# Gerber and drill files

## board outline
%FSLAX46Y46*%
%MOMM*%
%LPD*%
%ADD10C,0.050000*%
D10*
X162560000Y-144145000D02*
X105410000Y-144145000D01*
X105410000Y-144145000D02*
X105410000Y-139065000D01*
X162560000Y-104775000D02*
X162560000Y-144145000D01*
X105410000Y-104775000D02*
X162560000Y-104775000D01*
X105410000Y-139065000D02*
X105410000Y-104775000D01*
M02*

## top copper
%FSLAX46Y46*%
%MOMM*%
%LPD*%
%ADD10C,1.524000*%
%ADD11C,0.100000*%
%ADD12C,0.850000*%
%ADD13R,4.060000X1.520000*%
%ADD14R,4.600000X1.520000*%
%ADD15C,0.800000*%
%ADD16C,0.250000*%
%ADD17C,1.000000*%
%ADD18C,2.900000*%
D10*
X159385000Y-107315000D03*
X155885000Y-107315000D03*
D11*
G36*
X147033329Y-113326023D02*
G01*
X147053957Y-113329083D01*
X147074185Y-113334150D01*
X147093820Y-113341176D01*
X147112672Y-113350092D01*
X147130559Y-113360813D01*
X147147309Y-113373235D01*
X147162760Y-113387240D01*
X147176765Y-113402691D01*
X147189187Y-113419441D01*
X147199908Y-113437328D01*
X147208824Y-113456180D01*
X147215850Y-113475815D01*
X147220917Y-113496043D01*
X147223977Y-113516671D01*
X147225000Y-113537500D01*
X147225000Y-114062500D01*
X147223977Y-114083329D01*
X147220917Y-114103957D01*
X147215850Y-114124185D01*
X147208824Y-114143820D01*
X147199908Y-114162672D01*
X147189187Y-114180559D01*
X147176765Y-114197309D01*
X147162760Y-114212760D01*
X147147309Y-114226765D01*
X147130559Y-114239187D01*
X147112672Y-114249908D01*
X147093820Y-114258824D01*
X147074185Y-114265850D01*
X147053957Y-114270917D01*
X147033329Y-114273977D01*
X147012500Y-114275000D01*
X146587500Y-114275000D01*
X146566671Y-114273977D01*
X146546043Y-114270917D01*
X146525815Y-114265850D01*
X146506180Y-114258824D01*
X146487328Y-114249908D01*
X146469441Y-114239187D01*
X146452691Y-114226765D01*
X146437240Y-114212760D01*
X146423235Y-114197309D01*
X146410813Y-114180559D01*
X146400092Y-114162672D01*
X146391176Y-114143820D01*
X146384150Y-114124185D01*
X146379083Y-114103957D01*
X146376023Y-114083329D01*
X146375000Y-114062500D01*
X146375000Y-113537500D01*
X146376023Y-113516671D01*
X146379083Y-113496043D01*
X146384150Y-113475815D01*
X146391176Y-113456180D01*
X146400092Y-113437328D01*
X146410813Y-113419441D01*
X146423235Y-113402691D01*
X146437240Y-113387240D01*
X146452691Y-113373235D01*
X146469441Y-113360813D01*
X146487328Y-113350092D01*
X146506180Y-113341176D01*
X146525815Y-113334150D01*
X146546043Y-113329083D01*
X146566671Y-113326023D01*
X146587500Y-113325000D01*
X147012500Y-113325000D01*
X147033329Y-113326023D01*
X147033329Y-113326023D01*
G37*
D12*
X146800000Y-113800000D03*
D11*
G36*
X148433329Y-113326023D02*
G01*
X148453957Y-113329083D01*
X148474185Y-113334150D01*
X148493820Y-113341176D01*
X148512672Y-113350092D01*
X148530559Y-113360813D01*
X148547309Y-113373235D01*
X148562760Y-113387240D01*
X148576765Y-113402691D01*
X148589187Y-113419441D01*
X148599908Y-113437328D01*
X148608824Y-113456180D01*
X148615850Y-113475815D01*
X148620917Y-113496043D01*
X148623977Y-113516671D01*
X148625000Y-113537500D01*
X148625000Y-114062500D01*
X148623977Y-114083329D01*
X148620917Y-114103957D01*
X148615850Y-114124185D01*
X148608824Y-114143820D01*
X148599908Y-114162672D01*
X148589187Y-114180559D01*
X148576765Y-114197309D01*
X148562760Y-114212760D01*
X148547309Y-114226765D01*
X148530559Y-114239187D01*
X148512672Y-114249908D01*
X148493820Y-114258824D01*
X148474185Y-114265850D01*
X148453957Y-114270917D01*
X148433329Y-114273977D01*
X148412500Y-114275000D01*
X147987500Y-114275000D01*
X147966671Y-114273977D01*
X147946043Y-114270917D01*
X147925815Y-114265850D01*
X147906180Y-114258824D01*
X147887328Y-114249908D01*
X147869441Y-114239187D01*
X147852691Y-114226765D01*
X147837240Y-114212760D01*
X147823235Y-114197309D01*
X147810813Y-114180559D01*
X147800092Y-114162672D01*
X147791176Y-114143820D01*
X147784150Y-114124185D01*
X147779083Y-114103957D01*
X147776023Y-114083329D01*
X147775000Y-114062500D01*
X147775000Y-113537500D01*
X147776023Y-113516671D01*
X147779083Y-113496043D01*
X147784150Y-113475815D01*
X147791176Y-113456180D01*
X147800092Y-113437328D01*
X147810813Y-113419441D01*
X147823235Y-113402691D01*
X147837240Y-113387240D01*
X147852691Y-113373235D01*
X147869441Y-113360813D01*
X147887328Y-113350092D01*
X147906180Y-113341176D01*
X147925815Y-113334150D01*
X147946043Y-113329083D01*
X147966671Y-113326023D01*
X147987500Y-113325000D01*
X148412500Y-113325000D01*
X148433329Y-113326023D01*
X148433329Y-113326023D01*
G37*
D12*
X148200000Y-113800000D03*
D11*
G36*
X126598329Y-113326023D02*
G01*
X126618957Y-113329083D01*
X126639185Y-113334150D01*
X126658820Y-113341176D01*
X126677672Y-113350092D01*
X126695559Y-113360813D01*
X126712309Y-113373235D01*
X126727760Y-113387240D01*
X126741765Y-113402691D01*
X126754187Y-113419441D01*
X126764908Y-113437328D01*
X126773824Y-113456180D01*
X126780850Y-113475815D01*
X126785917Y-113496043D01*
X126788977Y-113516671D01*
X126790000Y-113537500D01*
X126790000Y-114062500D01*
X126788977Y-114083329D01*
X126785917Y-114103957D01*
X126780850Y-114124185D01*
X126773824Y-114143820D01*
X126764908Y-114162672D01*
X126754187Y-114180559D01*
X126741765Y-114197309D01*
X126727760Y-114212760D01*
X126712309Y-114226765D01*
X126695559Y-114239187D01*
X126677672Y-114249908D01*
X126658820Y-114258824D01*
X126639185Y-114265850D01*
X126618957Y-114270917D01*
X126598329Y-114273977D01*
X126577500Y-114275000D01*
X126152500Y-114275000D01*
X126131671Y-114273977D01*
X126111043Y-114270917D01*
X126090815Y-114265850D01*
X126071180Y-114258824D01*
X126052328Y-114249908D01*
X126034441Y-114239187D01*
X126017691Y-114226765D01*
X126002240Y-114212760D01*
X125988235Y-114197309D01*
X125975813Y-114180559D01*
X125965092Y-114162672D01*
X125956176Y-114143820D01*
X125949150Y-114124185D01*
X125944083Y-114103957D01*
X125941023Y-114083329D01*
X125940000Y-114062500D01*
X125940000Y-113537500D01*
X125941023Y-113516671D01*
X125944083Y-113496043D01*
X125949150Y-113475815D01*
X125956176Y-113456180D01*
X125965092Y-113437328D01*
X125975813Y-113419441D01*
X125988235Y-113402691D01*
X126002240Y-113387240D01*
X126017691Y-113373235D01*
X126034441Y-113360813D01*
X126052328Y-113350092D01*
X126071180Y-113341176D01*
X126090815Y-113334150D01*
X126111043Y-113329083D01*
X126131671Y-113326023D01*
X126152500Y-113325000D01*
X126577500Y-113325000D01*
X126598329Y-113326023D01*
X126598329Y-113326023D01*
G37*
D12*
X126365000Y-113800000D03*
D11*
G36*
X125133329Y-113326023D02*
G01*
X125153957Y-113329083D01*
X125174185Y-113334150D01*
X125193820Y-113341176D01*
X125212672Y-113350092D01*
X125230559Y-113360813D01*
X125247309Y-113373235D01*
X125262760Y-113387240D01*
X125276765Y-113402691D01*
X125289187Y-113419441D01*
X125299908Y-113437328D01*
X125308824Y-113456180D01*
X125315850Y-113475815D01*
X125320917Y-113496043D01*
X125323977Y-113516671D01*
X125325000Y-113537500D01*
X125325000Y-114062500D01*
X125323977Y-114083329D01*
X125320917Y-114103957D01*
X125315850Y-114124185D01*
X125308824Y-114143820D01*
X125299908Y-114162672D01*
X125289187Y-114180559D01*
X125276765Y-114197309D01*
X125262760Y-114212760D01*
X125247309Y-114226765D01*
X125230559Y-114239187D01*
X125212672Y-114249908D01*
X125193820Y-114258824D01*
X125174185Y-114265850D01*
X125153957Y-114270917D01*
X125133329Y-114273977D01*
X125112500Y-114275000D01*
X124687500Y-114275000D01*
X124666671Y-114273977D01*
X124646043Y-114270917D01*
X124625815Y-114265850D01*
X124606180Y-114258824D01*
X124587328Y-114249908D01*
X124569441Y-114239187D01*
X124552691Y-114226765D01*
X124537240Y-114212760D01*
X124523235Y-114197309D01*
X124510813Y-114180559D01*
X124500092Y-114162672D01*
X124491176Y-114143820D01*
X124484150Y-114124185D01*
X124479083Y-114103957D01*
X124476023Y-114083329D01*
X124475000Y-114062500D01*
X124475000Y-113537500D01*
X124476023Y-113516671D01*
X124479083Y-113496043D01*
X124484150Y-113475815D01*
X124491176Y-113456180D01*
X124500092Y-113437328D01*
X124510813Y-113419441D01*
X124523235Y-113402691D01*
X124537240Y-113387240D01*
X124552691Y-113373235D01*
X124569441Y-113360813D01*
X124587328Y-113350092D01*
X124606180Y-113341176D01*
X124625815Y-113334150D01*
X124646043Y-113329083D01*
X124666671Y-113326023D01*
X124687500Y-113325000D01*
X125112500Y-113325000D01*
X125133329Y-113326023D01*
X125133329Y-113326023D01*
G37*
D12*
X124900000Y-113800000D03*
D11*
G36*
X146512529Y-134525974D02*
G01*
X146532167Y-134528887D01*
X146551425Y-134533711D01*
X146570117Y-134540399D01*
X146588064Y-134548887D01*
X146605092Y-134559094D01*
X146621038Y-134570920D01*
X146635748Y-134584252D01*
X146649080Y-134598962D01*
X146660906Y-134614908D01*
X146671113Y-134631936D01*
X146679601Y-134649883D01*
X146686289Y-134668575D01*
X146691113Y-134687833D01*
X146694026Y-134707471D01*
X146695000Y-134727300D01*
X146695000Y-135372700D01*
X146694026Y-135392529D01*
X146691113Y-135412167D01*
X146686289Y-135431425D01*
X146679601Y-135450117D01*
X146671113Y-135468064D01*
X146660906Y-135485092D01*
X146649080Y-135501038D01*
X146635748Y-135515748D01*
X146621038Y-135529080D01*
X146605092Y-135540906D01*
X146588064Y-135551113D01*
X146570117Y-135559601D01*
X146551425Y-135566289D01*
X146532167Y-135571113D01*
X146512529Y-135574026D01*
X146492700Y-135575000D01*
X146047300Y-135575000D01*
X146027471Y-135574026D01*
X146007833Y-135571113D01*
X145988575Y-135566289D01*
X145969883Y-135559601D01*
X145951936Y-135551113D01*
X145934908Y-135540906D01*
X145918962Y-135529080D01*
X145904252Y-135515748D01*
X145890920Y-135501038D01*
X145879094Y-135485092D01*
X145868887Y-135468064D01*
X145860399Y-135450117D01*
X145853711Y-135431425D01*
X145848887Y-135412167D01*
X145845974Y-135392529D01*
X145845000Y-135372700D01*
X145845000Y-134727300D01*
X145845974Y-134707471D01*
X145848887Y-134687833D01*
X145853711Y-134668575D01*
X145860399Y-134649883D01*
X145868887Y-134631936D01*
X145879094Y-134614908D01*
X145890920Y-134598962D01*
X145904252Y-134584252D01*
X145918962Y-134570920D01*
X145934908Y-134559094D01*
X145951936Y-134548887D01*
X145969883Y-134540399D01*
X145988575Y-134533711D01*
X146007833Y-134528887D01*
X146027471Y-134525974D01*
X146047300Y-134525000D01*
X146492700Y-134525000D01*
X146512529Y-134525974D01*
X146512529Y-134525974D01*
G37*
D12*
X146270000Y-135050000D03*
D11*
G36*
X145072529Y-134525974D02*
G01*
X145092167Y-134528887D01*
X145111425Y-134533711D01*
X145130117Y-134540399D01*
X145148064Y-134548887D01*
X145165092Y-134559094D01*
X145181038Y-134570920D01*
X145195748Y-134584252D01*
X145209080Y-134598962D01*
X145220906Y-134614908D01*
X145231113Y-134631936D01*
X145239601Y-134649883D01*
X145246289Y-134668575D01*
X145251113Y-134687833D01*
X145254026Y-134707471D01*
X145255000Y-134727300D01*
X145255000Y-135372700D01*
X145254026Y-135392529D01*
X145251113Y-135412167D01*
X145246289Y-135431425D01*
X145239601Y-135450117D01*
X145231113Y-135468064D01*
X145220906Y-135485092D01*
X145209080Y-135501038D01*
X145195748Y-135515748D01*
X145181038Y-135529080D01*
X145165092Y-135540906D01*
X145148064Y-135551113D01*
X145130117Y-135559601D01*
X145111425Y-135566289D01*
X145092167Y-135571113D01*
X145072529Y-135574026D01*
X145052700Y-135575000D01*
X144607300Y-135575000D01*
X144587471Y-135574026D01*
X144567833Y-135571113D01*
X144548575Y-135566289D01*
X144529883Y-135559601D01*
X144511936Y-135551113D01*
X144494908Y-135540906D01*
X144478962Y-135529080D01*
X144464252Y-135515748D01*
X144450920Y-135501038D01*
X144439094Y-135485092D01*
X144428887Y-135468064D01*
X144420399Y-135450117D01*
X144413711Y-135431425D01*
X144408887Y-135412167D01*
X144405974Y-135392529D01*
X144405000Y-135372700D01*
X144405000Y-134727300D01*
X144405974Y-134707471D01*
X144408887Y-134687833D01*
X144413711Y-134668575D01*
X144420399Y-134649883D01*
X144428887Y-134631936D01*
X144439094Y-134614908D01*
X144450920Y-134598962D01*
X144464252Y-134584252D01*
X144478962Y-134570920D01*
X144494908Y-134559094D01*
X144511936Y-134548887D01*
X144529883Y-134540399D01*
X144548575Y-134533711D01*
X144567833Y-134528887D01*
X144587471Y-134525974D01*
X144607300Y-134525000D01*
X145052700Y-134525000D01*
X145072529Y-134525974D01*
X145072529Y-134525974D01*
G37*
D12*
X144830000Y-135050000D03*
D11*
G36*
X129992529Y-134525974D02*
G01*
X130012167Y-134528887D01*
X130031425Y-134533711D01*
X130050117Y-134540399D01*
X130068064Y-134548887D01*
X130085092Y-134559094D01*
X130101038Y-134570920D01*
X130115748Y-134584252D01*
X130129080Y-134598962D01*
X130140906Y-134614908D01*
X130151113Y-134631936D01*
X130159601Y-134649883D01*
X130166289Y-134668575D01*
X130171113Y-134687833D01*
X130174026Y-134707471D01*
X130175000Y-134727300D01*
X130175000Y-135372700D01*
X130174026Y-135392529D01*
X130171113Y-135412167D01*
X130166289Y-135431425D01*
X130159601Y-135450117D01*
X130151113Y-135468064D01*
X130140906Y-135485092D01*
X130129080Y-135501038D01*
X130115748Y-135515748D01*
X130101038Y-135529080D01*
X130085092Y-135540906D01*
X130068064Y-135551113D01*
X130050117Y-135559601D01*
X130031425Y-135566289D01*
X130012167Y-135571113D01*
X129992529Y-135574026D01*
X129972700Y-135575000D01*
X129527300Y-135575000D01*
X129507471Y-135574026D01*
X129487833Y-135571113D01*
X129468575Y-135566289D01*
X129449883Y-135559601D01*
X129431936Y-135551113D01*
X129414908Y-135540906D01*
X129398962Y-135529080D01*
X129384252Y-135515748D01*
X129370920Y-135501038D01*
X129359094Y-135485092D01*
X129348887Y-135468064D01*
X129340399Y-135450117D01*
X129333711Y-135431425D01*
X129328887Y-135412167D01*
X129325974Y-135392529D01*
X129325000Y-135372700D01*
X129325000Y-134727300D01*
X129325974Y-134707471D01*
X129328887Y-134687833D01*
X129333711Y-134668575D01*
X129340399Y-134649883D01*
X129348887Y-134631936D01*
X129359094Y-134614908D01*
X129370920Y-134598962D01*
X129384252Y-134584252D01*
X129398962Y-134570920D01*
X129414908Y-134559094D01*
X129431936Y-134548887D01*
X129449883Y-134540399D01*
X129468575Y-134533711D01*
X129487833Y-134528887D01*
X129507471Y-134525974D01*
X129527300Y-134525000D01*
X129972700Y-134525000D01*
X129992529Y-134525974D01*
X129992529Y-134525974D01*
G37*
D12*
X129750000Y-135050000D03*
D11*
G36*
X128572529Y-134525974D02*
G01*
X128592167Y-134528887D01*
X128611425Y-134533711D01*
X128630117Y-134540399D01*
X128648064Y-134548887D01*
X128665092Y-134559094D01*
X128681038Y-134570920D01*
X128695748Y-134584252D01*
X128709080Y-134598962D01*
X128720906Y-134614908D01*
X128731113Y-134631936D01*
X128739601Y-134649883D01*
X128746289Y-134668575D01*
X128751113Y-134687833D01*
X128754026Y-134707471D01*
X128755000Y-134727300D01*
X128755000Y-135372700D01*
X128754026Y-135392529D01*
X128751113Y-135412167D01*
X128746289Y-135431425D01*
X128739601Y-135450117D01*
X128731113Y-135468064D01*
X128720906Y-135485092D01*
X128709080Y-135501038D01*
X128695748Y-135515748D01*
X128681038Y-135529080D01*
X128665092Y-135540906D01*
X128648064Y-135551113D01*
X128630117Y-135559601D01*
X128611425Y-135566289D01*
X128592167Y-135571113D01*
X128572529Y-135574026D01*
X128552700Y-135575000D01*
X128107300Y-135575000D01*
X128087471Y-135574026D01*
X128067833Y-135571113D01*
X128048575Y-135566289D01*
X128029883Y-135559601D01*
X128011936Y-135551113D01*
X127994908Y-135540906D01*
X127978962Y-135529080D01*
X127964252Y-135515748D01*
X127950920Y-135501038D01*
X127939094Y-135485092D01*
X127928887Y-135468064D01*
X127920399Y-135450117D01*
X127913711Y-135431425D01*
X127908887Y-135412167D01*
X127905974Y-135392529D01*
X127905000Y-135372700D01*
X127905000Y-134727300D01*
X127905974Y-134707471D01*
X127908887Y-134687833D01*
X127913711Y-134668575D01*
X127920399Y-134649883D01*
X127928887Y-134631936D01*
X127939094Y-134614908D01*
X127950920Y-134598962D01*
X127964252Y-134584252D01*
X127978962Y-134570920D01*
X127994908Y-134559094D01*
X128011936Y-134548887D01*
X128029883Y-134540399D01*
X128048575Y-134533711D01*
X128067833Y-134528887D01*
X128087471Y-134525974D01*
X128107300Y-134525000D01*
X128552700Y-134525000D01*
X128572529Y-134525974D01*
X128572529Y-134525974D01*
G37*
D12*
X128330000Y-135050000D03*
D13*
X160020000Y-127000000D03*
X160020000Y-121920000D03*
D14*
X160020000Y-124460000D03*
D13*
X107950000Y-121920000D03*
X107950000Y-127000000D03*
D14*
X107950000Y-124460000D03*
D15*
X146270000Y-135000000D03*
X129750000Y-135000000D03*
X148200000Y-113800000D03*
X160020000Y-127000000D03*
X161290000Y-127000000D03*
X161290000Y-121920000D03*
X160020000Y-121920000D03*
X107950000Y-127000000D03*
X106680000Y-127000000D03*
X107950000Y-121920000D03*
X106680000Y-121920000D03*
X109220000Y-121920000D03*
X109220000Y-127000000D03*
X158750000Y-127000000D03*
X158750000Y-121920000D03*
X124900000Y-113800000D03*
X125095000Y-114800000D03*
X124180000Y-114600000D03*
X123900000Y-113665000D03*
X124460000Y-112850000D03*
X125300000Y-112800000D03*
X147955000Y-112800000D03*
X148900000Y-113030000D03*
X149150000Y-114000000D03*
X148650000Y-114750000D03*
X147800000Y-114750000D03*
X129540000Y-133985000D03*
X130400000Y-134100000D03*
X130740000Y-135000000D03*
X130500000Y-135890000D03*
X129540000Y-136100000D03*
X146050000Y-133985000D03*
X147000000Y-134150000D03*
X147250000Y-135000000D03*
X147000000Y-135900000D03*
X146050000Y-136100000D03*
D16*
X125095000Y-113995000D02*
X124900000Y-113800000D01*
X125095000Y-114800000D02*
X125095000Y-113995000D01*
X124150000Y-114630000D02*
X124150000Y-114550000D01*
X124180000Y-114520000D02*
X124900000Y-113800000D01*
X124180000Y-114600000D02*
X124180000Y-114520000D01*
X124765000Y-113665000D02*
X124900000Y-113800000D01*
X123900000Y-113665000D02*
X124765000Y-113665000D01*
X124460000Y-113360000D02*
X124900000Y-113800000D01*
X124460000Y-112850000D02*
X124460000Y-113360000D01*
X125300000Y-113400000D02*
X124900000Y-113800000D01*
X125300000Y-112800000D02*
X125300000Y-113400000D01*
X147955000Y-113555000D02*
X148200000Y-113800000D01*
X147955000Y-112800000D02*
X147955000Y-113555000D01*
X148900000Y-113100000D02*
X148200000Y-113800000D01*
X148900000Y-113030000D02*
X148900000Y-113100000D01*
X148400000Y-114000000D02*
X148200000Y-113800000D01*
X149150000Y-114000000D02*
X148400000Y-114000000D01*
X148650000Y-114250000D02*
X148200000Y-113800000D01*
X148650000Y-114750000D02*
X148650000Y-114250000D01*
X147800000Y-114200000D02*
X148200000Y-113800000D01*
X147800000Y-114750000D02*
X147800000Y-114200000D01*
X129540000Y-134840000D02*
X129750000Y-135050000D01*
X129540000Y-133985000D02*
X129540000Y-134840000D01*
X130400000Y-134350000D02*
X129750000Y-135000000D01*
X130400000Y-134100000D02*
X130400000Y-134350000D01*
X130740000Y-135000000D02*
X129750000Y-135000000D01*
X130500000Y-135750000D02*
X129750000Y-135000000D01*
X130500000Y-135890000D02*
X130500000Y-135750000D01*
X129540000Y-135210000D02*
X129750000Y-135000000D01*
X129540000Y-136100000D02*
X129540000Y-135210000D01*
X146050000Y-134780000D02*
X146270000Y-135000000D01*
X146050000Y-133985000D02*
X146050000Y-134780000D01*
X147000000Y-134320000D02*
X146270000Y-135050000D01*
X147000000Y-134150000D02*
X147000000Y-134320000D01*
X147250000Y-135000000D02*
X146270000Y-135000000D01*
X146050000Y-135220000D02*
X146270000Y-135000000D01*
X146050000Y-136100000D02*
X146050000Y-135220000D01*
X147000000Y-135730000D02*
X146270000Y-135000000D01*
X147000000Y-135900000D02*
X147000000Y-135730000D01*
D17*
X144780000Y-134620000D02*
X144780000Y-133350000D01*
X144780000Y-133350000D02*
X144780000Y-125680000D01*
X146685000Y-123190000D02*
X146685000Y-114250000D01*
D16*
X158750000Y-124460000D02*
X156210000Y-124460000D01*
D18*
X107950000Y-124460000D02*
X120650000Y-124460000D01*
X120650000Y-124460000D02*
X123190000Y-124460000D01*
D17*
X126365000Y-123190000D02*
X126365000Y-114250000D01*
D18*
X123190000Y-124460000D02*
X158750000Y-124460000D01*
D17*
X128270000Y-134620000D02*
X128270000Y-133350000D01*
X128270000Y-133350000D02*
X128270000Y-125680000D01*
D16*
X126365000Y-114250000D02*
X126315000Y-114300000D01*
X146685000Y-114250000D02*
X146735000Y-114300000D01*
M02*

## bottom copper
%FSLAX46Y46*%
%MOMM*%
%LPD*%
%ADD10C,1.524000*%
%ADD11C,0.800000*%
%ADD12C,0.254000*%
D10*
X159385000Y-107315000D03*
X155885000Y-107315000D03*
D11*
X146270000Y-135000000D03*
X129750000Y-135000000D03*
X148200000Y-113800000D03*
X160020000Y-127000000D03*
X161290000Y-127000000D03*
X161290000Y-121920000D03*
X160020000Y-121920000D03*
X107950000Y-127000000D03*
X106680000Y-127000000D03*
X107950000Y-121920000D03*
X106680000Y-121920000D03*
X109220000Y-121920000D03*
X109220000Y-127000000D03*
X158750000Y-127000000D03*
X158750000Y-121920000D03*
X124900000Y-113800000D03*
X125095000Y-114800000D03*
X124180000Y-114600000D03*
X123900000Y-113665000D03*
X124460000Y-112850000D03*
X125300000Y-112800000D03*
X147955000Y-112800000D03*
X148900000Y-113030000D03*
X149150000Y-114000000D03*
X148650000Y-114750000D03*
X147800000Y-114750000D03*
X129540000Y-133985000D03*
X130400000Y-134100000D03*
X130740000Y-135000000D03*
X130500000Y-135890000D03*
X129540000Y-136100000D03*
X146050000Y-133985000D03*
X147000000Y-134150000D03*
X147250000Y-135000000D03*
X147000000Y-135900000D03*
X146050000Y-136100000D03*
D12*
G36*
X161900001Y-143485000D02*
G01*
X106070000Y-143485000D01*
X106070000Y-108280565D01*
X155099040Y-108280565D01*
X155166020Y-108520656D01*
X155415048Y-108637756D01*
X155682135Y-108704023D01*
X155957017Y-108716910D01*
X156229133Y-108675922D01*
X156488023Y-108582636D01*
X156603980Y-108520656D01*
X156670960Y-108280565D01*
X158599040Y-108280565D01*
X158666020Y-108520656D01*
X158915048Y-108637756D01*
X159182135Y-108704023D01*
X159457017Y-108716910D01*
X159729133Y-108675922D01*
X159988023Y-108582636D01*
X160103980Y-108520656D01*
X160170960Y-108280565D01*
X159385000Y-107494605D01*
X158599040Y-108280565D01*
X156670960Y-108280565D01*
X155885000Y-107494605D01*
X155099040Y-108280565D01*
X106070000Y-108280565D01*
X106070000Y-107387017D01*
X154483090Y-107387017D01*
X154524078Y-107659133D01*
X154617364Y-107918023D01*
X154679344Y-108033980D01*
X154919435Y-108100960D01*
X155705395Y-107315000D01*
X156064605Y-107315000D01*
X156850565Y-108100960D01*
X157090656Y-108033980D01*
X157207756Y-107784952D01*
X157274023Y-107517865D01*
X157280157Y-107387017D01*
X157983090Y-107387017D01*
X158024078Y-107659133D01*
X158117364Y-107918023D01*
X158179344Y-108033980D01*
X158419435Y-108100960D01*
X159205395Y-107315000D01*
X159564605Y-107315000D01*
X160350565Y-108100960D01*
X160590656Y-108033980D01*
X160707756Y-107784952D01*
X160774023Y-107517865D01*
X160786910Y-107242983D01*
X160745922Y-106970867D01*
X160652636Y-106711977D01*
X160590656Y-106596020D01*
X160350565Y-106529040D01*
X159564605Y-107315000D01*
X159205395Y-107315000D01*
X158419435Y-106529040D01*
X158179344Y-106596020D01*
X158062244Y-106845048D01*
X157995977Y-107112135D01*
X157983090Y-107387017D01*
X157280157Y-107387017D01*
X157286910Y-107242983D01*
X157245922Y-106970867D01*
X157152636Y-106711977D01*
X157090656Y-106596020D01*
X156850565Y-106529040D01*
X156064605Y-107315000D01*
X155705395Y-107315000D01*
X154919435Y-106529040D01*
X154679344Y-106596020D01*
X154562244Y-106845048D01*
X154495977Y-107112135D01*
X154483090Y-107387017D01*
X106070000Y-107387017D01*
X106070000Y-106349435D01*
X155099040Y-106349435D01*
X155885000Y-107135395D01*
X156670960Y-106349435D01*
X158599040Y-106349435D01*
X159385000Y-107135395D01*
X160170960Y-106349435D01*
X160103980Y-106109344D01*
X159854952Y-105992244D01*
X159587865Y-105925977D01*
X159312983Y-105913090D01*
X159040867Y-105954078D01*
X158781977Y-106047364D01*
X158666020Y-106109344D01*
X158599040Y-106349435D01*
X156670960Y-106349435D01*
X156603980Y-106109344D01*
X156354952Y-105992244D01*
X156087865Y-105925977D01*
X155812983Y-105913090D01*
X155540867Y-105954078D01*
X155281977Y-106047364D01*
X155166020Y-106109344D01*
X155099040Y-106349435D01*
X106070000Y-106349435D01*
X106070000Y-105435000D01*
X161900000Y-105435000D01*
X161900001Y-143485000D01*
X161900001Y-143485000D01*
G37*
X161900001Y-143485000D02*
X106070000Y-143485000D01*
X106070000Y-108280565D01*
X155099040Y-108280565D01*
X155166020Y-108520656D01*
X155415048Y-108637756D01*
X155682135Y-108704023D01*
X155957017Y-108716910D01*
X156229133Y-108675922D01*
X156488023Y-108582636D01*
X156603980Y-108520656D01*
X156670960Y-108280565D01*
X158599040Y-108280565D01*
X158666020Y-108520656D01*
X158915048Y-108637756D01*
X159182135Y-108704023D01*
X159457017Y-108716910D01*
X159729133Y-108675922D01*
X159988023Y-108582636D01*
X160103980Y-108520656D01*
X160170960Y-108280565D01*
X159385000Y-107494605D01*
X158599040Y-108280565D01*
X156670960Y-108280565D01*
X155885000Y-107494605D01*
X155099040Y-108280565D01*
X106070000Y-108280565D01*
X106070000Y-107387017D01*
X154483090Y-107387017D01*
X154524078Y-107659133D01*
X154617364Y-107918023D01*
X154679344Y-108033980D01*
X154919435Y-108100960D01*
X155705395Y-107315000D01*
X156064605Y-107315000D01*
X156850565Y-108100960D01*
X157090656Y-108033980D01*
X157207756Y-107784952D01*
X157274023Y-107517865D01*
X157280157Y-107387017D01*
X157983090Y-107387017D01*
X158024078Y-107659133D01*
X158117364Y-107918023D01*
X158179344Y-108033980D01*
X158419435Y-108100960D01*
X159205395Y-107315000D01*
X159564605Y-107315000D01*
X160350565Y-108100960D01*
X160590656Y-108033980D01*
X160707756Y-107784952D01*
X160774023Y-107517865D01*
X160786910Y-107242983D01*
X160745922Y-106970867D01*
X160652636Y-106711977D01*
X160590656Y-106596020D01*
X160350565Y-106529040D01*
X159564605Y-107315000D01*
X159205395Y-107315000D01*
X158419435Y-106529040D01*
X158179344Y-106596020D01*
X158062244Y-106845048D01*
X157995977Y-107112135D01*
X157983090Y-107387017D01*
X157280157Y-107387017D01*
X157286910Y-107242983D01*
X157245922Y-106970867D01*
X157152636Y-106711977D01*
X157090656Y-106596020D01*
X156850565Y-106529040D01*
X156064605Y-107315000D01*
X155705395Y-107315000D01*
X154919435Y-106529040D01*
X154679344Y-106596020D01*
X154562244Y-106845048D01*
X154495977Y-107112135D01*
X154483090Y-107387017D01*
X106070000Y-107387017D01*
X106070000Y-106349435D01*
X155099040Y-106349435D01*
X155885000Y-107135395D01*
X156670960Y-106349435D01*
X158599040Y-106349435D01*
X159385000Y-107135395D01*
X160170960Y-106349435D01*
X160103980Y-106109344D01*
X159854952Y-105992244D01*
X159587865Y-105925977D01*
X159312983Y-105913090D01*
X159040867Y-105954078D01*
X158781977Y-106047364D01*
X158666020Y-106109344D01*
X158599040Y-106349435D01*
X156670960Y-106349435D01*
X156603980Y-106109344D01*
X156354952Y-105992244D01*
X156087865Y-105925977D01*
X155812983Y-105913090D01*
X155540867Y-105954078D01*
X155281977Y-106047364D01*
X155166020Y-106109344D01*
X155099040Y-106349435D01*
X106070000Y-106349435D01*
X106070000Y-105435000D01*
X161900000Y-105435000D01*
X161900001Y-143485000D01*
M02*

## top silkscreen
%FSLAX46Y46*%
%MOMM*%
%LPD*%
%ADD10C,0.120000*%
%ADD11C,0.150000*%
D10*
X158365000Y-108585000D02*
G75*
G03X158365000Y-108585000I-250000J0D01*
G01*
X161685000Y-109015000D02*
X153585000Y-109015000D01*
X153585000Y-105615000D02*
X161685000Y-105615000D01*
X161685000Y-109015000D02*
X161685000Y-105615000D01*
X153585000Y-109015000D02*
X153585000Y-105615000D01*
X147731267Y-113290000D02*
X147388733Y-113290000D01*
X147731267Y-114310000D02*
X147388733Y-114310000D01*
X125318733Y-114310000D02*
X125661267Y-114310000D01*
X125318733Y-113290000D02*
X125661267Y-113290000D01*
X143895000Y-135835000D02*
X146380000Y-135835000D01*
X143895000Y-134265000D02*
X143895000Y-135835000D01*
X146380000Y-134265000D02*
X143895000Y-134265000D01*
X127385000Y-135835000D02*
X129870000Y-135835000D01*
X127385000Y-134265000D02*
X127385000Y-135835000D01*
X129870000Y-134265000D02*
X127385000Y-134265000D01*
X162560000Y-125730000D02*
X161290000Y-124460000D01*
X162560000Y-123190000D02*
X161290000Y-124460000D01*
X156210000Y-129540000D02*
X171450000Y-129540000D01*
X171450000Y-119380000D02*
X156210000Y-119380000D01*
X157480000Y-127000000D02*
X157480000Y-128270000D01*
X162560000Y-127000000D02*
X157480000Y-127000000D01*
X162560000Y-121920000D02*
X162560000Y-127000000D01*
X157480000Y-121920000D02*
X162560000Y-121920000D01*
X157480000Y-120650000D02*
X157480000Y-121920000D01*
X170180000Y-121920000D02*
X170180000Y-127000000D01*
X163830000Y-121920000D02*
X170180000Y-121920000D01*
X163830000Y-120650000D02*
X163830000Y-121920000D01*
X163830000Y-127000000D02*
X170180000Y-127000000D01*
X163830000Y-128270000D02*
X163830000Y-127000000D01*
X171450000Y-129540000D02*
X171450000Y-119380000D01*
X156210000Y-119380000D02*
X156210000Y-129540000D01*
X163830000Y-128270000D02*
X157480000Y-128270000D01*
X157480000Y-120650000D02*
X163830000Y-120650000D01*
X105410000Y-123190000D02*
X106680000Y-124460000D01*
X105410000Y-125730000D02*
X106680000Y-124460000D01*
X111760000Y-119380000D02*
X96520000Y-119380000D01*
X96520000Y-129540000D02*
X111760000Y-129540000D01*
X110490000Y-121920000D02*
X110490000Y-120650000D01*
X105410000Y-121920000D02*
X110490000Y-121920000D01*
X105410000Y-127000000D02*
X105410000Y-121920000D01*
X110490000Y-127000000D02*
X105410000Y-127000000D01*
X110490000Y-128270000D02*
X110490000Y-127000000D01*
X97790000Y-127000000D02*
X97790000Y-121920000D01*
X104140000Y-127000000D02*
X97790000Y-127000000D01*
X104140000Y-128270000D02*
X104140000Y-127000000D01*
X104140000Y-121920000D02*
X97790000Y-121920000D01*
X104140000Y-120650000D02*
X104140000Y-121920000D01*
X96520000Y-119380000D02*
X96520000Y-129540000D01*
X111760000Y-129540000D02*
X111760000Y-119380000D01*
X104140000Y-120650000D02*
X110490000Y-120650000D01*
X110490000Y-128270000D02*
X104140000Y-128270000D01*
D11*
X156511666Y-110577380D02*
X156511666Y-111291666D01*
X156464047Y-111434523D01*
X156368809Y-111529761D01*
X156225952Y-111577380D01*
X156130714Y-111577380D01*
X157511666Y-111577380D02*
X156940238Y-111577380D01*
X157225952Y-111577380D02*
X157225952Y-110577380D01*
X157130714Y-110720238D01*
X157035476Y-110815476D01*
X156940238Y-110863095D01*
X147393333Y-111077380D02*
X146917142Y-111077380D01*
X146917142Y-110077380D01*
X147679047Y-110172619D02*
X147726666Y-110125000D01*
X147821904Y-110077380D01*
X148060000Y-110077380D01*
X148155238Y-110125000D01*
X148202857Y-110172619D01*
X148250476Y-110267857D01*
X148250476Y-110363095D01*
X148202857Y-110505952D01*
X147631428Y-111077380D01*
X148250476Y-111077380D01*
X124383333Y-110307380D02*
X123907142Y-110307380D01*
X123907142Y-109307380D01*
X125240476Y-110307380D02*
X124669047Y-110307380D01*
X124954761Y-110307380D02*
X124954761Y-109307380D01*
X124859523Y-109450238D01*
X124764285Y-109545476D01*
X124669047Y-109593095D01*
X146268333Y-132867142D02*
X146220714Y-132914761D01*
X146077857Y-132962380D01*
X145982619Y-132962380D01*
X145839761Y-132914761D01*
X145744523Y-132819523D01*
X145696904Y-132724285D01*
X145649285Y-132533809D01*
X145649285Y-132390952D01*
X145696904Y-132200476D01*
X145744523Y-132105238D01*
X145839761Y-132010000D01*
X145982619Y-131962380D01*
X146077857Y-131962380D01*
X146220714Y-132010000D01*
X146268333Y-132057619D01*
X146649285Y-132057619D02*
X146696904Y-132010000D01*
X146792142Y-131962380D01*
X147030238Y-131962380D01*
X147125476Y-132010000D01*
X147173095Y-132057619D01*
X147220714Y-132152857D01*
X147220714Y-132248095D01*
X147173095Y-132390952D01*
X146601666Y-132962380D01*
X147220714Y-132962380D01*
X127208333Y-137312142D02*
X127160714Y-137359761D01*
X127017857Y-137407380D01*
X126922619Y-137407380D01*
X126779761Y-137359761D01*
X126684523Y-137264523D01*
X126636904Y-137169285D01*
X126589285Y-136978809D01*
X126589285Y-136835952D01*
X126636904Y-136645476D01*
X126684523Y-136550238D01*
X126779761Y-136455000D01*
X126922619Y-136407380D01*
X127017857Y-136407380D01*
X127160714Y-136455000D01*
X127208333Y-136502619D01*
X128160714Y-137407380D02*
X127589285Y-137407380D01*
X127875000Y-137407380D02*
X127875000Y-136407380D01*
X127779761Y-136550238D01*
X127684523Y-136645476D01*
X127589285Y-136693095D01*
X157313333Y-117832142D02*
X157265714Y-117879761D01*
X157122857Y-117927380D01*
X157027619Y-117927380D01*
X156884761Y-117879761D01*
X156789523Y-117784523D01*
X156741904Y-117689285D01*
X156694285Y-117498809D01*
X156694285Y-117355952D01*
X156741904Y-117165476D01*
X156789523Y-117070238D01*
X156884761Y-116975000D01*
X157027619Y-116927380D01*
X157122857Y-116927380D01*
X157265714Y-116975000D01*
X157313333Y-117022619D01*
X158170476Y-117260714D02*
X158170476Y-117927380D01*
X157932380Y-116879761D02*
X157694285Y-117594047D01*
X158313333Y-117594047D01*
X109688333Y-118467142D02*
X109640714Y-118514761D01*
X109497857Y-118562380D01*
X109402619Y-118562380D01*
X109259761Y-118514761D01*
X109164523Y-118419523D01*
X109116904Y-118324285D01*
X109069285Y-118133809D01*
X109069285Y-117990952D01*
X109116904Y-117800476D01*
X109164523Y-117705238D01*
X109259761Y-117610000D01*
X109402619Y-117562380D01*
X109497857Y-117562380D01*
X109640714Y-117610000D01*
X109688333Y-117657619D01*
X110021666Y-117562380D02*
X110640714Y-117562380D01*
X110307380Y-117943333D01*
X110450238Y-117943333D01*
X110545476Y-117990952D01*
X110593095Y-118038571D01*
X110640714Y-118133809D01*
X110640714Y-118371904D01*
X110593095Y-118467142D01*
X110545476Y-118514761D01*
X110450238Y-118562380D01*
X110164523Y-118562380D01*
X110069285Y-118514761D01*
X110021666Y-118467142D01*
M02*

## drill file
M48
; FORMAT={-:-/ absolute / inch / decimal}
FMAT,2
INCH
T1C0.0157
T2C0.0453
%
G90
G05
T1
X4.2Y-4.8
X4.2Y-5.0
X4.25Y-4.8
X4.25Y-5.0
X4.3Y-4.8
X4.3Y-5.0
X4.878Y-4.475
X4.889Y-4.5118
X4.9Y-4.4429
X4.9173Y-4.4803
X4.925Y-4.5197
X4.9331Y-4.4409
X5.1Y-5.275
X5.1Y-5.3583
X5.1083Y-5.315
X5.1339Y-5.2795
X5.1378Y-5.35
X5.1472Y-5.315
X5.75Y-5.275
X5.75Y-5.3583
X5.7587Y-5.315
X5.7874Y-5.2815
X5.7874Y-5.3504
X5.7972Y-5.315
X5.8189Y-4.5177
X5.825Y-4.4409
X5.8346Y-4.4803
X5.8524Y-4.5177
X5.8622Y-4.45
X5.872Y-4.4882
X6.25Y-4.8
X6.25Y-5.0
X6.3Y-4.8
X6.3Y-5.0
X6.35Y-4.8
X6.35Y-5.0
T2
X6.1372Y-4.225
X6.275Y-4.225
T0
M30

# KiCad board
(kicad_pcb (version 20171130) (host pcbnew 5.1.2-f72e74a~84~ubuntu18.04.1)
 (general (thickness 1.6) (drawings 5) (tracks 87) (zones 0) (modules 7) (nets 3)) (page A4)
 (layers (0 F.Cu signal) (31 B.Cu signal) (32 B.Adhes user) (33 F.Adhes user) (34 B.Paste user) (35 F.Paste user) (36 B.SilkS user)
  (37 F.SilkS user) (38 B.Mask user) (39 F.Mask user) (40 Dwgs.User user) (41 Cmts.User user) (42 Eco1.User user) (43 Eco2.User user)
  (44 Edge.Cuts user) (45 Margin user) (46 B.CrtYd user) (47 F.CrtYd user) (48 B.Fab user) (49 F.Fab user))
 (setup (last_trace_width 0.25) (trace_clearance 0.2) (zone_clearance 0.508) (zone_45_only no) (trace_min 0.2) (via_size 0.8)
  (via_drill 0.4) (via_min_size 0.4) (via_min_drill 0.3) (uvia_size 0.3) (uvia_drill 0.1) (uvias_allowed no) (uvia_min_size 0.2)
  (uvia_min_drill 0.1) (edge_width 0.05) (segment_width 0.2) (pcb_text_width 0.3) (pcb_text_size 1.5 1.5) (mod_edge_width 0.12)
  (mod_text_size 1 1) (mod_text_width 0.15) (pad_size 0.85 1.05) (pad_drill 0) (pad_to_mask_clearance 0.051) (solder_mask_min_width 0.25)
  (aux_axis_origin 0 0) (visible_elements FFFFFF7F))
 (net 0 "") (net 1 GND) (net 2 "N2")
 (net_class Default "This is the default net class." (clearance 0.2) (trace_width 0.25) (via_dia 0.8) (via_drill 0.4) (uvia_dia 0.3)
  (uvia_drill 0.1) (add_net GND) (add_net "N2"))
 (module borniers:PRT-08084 (layer F.Cu) (at 159.385 112.395)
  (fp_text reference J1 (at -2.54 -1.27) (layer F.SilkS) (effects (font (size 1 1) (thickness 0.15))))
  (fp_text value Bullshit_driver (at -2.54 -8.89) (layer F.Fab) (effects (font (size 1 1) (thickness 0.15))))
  (fp_circle (center -1.27 -3.81) (end -1.02 -3.81) (layer F.SilkS) (width 0.12))
  (fp_line (start 2.3 -3.38) (end -5.8 -3.38) (layer F.SilkS) (width 0.12))
  (fp_line (start -5.8 -6.78) (end 2.3 -6.78) (layer F.SilkS) (width 0.12))
  (fp_line (start 2.3 -3.38) (end 2.3 -6.78) (layer F.SilkS) (width 0.12))
  (fp_line (start -5.8 -3.38) (end -5.8 -6.78) (layer F.SilkS) (width 0.12))
  (pad 2 thru_hole circle (at 0 -5.08) (size 1.524 1.524) (drill 1.15) (layers *.Cu *.Mask) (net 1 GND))
  (pad 1 thru_hole circle (at -3.5 -5.08) (size 1.524 1.524) (drill 1.15) (layers *.Cu *.Mask) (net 1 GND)))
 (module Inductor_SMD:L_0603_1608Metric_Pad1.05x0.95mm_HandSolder (layer F.Cu) (at 147.56 113.8 180)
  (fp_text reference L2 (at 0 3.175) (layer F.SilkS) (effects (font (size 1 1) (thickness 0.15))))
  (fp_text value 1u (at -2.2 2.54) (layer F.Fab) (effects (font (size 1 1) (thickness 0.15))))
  (fp_line (start -0.171267 0.51) (end 0.171267 0.51) (layer F.SilkS) (width 0.12))
  (fp_line (start -0.171267 -0.51) (end 0.171267 -0.51) (layer F.SilkS) (width 0.12))
  (pad 2 smd roundrect (at 0.76 0 180) (size 0.85 0.95) (layers F.Cu F.Paste F.Mask) (roundrect_rratio 0.25) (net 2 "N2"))
  (pad 1 smd roundrect (at -0.64 0 180) (size 0.85 0.95) (layers F.Cu F.Paste F.Mask) (roundrect_rratio 0.25) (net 1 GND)))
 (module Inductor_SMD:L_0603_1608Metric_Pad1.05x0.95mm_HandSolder (layer F.Cu) (at 125.49 113.8)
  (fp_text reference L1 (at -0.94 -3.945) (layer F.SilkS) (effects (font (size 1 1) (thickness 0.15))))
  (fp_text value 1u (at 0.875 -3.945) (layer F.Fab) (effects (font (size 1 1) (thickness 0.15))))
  (fp_line (start -0.171267 0.51) (end 0.171267 0.51) (layer F.SilkS) (width 0.12))
  (fp_line (start -0.171267 -0.51) (end 0.171267 -0.51) (layer F.SilkS) (width 0.12))
  (pad 2 smd roundrect (at 0.875 0) (size 0.85 0.95) (layers F.Cu F.Paste F.Mask) (roundrect_rratio 0.25) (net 2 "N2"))
  (pad 1 smd roundrect (at -0.59 0) (size 0.85 0.95) (layers F.Cu F.Paste F.Mask) (roundrect_rratio 0.25) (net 1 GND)))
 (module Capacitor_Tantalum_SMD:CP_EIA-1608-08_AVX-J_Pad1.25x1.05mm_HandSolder (layer F.Cu) (at 145.58 135.05)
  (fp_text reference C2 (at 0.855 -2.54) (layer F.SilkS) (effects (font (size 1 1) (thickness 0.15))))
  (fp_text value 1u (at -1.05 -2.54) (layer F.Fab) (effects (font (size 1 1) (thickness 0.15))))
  (fp_line (start -1.685 0.785) (end 0.8 0.785) (layer F.SilkS) (width 0.12))
  (fp_line (start -1.685 -0.785) (end -1.685 0.785) (layer F.SilkS) (width 0.12))
  (fp_line (start 0.8 -0.785) (end -1.685 -0.785) (layer F.SilkS) (width 0.12))
  (pad 2 smd roundrect (at 0.69 0) (size 0.85 1.05) (layers F.Cu F.Paste F.Mask) (roundrect_rratio 0.238) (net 1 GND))
  (pad 1 smd roundrect (at -0.75 0) (size 0.85 1.05) (layers F.Cu F.Paste F.Mask) (roundrect_rratio 0.238) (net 2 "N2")))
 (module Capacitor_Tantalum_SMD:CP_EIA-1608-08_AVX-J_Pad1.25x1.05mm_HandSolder (layer F.Cu) (at 129.07 135.05)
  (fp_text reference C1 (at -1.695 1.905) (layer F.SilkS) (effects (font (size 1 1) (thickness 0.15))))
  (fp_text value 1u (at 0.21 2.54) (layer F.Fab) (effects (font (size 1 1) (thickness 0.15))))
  (fp_line (start -1.685 0.785) (end 0.8 0.785) (layer F.SilkS) (width 0.12))
  (fp_line (start -1.685 -0.785) (end -1.685 0.785) (layer F.SilkS) (width 0.12))
  (fp_line (start 0.8 -0.785) (end -1.685 -0.785) (layer F.SilkS) (width 0.12))
  (pad 2 smd roundrect (at 0.68 0) (size 0.85 1.05) (layers F.Cu F.Paste F.Mask) (roundrect_rratio 0.238) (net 1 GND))
  (pad 1 smd roundrect (at -0.74 0) (size 0.85 1.05) (layers F.Cu F.Paste F.Mask) (roundrect_rratio 0.238) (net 2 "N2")))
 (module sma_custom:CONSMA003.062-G (layer F.Cu) (at 163.83 127)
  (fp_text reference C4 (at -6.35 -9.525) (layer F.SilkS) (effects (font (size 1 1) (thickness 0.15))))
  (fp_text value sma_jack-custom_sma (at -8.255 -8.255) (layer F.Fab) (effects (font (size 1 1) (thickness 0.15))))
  (fp_line (start -1.27 -1.27) (end -2.54 -2.54) (layer F.SilkS) (width 0.12))
  (fp_line (start -1.27 -3.81) (end -2.54 -2.54) (layer F.SilkS) (width 0.12))
  (fp_line (start -7.62 2.54) (end 7.62 2.54) (layer F.SilkS) (width 0.12))
  (fp_line (start 7.62 -7.62) (end -7.62 -7.62) (layer F.SilkS) (width 0.12))
  (fp_line (start -6.35 0) (end -6.35 1.27) (layer F.SilkS) (width 0.12))
  (fp_line (start -1.27 0) (end -6.35 0) (layer F.SilkS) (width 0.12))
  (fp_line (start -1.27 -5.08) (end -1.27 0) (layer F.SilkS) (width 0.12))
  (fp_line (start -6.35 -5.08) (end -1.27 -5.08) (layer F.SilkS) (width 0.12))
  (fp_line (start -6.35 -6.35) (end -6.35 -5.08) (layer F.SilkS) (width 0.12))
  (fp_line (start 6.35 -5.08) (end 6.35 0) (layer F.SilkS) (width 0.12))
  (fp_line (start 0 -5.08) (end 6.35 -5.08) (layer F.SilkS) (width 0.12))
  (fp_line (start 0 -6.35) (end 0 -5.08) (layer F.SilkS) (width 0.12))
  (fp_line (start 0 0) (end 6.35 0) (layer F.SilkS) (width 0.12))
  (fp_line (start 0 1.27) (end 0 0) (layer F.SilkS) (width 0.12))
  (fp_line (start 7.62 2.54) (end 7.62 -7.62) (layer F.SilkS) (width 0.12))
  (fp_line (start -7.62 -7.62) (end -7.62 2.54) (layer F.SilkS) (width 0.12))
  (fp_line (start 0 1.27) (end -6.35 1.27) (layer F.SilkS) (width 0.12))
  (fp_line (start -6.35 -6.35) (end 0 -6.35) (layer F.SilkS) (width 0.12))
  (pad 3 smd rect (at -3.81 0) (size 4.06 1.52) (layers F.Cu F.Paste F.Mask) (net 1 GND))
  (pad 2 smd rect (at -3.81 -5.08) (size 4.06 1.52) (layers F.Cu F.Paste F.Mask) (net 1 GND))
  (pad 1 smd rect (at -3.81 -2.54) (size 4.6 1.52) (layers F.Cu F.Paste F.Mask) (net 2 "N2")))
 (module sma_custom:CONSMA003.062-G (layer F.Cu) (at 104.14 121.92 180)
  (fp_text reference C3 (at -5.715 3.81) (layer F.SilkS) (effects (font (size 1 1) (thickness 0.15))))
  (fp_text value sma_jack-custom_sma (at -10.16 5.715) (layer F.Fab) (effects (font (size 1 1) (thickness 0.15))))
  (fp_line (start -1.27 -1.27) (end -2.54 -2.54) (layer F.SilkS) (width 0.12))
  (fp_line (start -1.27 -3.81) (end -2.54 -2.54) (layer F.SilkS) (width 0.12))
  (fp_line (start -7.62 2.54) (end 7.62 2.54) (layer F.SilkS) (width 0.12))
  (fp_line (start 7.62 -7.62) (end -7.62 -7.62) (layer F.SilkS) (width 0.12))
  (fp_line (start -6.35 0) (end -6.35 1.27) (layer F.SilkS) (width 0.12))
  (fp_line (start -1.27 0) (end -6.35 0) (layer F.SilkS) (width 0.12))
  (fp_line (start -1.27 -5.08) (end -1.27 0) (layer F.SilkS) (width 0.12))
  (fp_line (start -6.35 -5.08) (end -1.27 -5.08) (layer F.SilkS) (width 0.12))
  (fp_line (start -6.35 -6.35) (end -6.35 -5.08) (layer F.SilkS) (width 0.12))
  (fp_line (start 6.35 -5.08) (end 6.35 0) (layer F.SilkS) (width 0.12))
  (fp_line (start 0 -5.08) (end 6.35 -5.08) (layer F.SilkS) (width 0.12))
  (fp_line (start 0 -6.35) (end 0 -5.08) (layer F.SilkS) (width 0.12))
  (fp_line (start 0 0) (end 6.35 0) (layer F.SilkS) (width 0.12))
  (fp_line (start 0 1.27) (end 0 0) (layer F.SilkS) (width 0.12))
  (fp_line (start 7.62 2.54) (end 7.62 -7.62) (layer F.SilkS) (width 0.12))
  (fp_line (start -7.62 -7.62) (end -7.62 2.54) (layer F.SilkS) (width 0.12))
  (fp_line (start 0 1.27) (end -6.35 1.27) (layer F.SilkS) (width 0.12))
  (fp_line (start -6.35 -6.35) (end 0 -6.35) (layer F.SilkS) (width 0.12))
  (pad 3 smd rect (at -3.81 0 180) (size 4.06 1.52) (layers F.Cu F.Paste F.Mask) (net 1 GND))
  (pad 2 smd rect (at -3.81 -5.08 180) (size 4.06 1.52) (layers F.Cu F.Paste F.Mask) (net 1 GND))
  (pad 1 smd rect (at -3.81 -2.54 180) (size 4.6 1.52) (layers F.Cu F.Paste F.Mask) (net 2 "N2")))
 (gr_line (start 162.56 144.145) (end 105.41 144.145) (layer Edge.Cuts) (width 0.05))
 (gr_line (start 105.41 144.145) (end 105.41 139.065) (layer Edge.Cuts) (width 0.05))
 (gr_line (start 162.56 104.775) (end 162.56 144.145) (layer Edge.Cuts) (width 0.05))
 (gr_line (start 105.41 104.775) (end 162.56 104.775) (layer Edge.Cuts) (width 0.05))
 (gr_line (start 105.41 139.065) (end 105.41 104.775) (layer Edge.Cuts) (width 0.05))
 (via (at 146.27 135) (size 0.8) (drill 0.4) (layers F.Cu B.Cu) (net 1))
 (via (at 129.75 135) (size 0.8) (drill 0.4) (layers F.Cu B.Cu) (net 1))
 (via (at 148.2 113.8) (size 0.8) (drill 0.4) (layers F.Cu B.Cu) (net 1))
 (via (at 160.02 127) (size 0.8) (drill 0.4) (layers F.Cu B.Cu) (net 1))
 (via (at 161.29 127) (size 0.8) (drill 0.4) (layers F.Cu B.Cu) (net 1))
 (via (at 161.29 121.92) (size 0.8) (drill 0.4) (layers F.Cu B.Cu) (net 1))
 (via (at 160.02 121.92) (size 0.8) (drill 0.4) (layers F.Cu B.Cu) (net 1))
 (via (at 107.95 127) (size 0.8) (drill 0.4) (layers F.Cu B.Cu) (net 1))
 (via (at 106.68 127) (size 0.8) (drill 0.4) (layers F.Cu B.Cu) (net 1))
 (via (at 107.95 121.92) (size 0.8) (drill 0.4) (layers F.Cu B.Cu) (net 1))
 (via (at 106.68 121.92) (size 0.8) (drill 0.4) (layers F.Cu B.Cu) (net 1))
 (via (at 109.22 121.92) (size 0.8) (drill 0.4) (layers F.Cu B.Cu) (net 1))
 (via (at 109.22 127) (size 0.8) (drill 0.4) (layers F.Cu B.Cu) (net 1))
 (via (at 158.75 127) (size 0.8) (drill 0.4) (layers F.Cu B.Cu) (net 1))
 (via (at 158.75 121.92) (size 0.8) (drill 0.4) (layers F.Cu B.Cu) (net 1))
 (via (at 124.9 113.8) (size 0.8) (drill 0.4) (layers F.Cu B.Cu) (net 1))
 (via (at 125.095 114.8) (size 0.8) (drill 0.4) (layers F.Cu B.Cu) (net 1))
 (segment (start 125.095 113.995) (end 124.9 113.8) (width 0.25) (layer F.Cu) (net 1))
 (segment (start 125.095 114.8) (end 125.095 113.995) (width 0.25) (layer F.Cu) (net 1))
 (via (at 124.18 114.6) (size 0.8) (drill 0.4) (layers F.Cu B.Cu) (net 1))
 (segment (start 124.15 114.63) (end 124.15 114.55) (width 0.25) (layer F.Cu) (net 1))
 (segment (start 124.18 114.52) (end 124.9 113.8) (width 0.25) (layer F.Cu) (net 1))
 (segment (start 124.18 114.6) (end 124.18 114.52) (width 0.25) (layer F.Cu) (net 1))
 (via (at 123.9 113.665) (size 0.8) (drill 0.4) (layers F.Cu B.Cu) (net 1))
 (segment (start 124.765 113.665) (end 124.9 113.8) (width 0.25) (layer F.Cu) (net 1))
 (segment (start 123.9 113.665) (end 124.765 113.665) (width 0.25) (layer F.Cu) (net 1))
 (via (at 124.46 112.85) (size 0.8) (drill 0.4) (layers F.Cu B.Cu) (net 1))
 (segment (start 124.46 113.36) (end 124.9 113.8) (width 0.25) (layer F.Cu) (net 1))
 (segment (start 124.46 112.85) (end 124.46 113.36) (width 0.25) (layer F.Cu) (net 1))
 (via (at 125.3 112.8) (size 0.8) (drill 0.4) (layers F.Cu B.Cu) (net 1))
 (segment (start 125.3 113.4) (end 124.9 113.8) (width 0.25) (layer F.Cu) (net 1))
 (segment (start 125.3 112.8) (end 125.3 113.4) (width 0.25) (layer F.Cu) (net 1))
 (via (at 147.955 112.8) (size 0.8) (drill 0.4) (layers F.Cu B.Cu) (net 1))
 (via (at 148.9 113.03) (size 0.8) (drill 0.4) (layers F.Cu B.Cu) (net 1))
 (via (at 149.15 114) (size 0.8) (drill 0.4) (layers F.Cu B.Cu) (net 1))
 (via (at 148.65 114.75) (size 0.8) (drill 0.4) (layers F.Cu B.Cu) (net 1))
 (segment (start 147.955 113.555) (end 148.2 113.8) (width 0.25) (layer F.Cu) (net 1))
 (segment (start 147.955 112.8) (end 147.955 113.555) (width 0.25) (layer F.Cu) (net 1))
 (segment (start 148.9 113.1) (end 148.2 113.8) (width 0.25) (layer F.Cu) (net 1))
 (segment (start 148.9 113.03) (end 148.9 113.1) (width 0.25) (layer F.Cu) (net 1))
 (segment (start 148.4 114) (end 148.2 113.8) (width 0.25) (layer F.Cu) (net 1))
 (segment (start 149.15 114) (end 148.4 114) (width 0.25) (layer F.Cu) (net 1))
 (segment (start 148.65 114.25) (end 148.2 113.8) (width 0.25) (layer F.Cu) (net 1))
 (segment (start 148.65 114.75) (end 148.65 114.25) (width 0.25) (layer F.Cu) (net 1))
 (via (at 147.8 114.75) (size 0.8) (drill 0.4) (layers F.Cu B.Cu) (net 1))
 (segment (start 147.8 114.2) (end 148.2 113.8) (width 0.25) (layer F.Cu) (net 1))
 (segment (start 147.8 114.75) (end 147.8 114.2) (width 0.25) (layer F.Cu) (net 1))
 (via (at 129.54 133.985) (size 0.8) (drill 0.4) (layers F.Cu B.Cu) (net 1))
 (via (at 130.4 134.1) (size 0.8) (drill 0.4) (layers F.Cu B.Cu) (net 1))
 (via (at 130.74 135) (size 0.8) (drill 0.4) (layers F.Cu B.Cu) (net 1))
 (via (at 130.5 135.89) (size 0.8) (drill 0.4) (layers F.Cu B.Cu) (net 1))
 (via (at 129.54 136.1) (size 0.8) (drill 0.4) (layers F.Cu B.Cu) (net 1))
 (segment (start 129.54 134.84) (end 129.75 135.05) (width 0.25) (layer F.Cu) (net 1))
 (segment (start 129.54 133.985) (end 129.54 134.84) (width 0.25) (layer F.Cu) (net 1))
 (segment (start 130.4 134.35) (end 129.75 135) (width 0.25) (layer F.Cu) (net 1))
 (segment (start 130.4 134.1) (end 130.4 134.35) (width 0.25) (layer F.Cu) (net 1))
 (segment (start 130.74 135) (end 129.75 135) (width 0.25) (layer F.Cu) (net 1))
 (segment (start 130.5 135.75) (end 129.75 135) (width 0.25) (layer F.Cu) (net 1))
 (segment (start 130.5 135.89) (end 130.5 135.75) (width 0.25) (layer F.Cu) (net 1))
 (segment (start 129.54 135.21) (end 129.75 135) (width 0.25) (layer F.Cu) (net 1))
 (segment (start 129.54 136.1) (end 129.54 135.21) (width 0.25) (layer F.Cu) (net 1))
 (via (at 146.05 133.985) (size 0.8) (drill 0.4) (layers F.Cu B.Cu) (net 1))
 (via (at 147 134.15) (size 0.8) (drill 0.4) (layers F.Cu B.Cu) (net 1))
 (via (at 147.25 135) (size 0.8) (drill 0.4) (layers F.Cu B.Cu) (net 1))
 (via (at 147 135.9) (size 0.8) (drill 0.4) (layers F.Cu B.Cu) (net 1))
 (via (at 146.05 136.1) (size 0.8) (drill 0.4) (layers F.Cu B.Cu) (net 1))
 (segment (start 146.05 134.78) (end 146.27 135) (width 0.25) (layer F.Cu) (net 1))
 (segment (start 146.05 133.985) (end 146.05 134.78) (width 0.25) (layer F.Cu) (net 1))
 (segment (start 147 134.32) (end 146.27 135.05) (width 0.25) (layer F.Cu) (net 1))
 (segment (start 147 134.15) (end 147 134.32) (width 0.25) (layer F.Cu) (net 1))
 (segment (start 147.25 135) (end 146.27 135) (width 0.25) (layer F.Cu) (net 1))
 (segment (start 146.05 135.22) (end 146.27 135) (width 0.25) (layer F.Cu) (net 1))
 (segment (start 146.05 136.1) (end 146.05 135.22) (width 0.25) (layer F.Cu) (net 1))
 (segment (start 147 135.73) (end 146.27 135) (width 0.25) (layer F.Cu) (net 1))
 (segment (start 147 135.9) (end 147 135.73) (width 0.25) (layer F.Cu) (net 1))
 (segment (start 144.78 134.62) (end 144.78 133.35) (width 1) (layer F.Cu) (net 2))
 (segment (start 144.78 133.35) (end 144.78 125.68) (width 1) (layer F.Cu) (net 2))
 (segment (start 146.685 123.19) (end 146.685 114.25) (width 1) (layer F.Cu) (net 2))
 (segment (start 158.75 124.46) (end 156.21 124.46) (width 0.25) (layer F.Cu) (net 2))
 (segment (start 107.95 124.46) (end 120.65 124.46) (width 2.9) (layer F.Cu) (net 2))
 (segment (start 120.65 124.46) (end 123.19 124.46) (width 2.9) (layer F.Cu) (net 2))
 (segment (start 126.365 123.19) (end 126.365 114.25) (width 1) (layer F.Cu) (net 2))
 (segment (start 123.19 124.46) (end 158.75 124.46) (width 2.9) (layer F.Cu) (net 2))
 (segment (start 128.27 134.62) (end 128.27 133.35) (width 1) (layer F.Cu) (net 2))
 (segment (start 128.27 133.35) (end 128.27 125.68) (width 1) (layer F.Cu) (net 2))
 (segment (start 126.365 114.25) (end 126.315 114.3) (width 0.25) (layer F.Cu) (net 2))
 (segment (start 146.685 114.25) (end 146.735 114.3) (width 0.25) (layer F.Cu) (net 2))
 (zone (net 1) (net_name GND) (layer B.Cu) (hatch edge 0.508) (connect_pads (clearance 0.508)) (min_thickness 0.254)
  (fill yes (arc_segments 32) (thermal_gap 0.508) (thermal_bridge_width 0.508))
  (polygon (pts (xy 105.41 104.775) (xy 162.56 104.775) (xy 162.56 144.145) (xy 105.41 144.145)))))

